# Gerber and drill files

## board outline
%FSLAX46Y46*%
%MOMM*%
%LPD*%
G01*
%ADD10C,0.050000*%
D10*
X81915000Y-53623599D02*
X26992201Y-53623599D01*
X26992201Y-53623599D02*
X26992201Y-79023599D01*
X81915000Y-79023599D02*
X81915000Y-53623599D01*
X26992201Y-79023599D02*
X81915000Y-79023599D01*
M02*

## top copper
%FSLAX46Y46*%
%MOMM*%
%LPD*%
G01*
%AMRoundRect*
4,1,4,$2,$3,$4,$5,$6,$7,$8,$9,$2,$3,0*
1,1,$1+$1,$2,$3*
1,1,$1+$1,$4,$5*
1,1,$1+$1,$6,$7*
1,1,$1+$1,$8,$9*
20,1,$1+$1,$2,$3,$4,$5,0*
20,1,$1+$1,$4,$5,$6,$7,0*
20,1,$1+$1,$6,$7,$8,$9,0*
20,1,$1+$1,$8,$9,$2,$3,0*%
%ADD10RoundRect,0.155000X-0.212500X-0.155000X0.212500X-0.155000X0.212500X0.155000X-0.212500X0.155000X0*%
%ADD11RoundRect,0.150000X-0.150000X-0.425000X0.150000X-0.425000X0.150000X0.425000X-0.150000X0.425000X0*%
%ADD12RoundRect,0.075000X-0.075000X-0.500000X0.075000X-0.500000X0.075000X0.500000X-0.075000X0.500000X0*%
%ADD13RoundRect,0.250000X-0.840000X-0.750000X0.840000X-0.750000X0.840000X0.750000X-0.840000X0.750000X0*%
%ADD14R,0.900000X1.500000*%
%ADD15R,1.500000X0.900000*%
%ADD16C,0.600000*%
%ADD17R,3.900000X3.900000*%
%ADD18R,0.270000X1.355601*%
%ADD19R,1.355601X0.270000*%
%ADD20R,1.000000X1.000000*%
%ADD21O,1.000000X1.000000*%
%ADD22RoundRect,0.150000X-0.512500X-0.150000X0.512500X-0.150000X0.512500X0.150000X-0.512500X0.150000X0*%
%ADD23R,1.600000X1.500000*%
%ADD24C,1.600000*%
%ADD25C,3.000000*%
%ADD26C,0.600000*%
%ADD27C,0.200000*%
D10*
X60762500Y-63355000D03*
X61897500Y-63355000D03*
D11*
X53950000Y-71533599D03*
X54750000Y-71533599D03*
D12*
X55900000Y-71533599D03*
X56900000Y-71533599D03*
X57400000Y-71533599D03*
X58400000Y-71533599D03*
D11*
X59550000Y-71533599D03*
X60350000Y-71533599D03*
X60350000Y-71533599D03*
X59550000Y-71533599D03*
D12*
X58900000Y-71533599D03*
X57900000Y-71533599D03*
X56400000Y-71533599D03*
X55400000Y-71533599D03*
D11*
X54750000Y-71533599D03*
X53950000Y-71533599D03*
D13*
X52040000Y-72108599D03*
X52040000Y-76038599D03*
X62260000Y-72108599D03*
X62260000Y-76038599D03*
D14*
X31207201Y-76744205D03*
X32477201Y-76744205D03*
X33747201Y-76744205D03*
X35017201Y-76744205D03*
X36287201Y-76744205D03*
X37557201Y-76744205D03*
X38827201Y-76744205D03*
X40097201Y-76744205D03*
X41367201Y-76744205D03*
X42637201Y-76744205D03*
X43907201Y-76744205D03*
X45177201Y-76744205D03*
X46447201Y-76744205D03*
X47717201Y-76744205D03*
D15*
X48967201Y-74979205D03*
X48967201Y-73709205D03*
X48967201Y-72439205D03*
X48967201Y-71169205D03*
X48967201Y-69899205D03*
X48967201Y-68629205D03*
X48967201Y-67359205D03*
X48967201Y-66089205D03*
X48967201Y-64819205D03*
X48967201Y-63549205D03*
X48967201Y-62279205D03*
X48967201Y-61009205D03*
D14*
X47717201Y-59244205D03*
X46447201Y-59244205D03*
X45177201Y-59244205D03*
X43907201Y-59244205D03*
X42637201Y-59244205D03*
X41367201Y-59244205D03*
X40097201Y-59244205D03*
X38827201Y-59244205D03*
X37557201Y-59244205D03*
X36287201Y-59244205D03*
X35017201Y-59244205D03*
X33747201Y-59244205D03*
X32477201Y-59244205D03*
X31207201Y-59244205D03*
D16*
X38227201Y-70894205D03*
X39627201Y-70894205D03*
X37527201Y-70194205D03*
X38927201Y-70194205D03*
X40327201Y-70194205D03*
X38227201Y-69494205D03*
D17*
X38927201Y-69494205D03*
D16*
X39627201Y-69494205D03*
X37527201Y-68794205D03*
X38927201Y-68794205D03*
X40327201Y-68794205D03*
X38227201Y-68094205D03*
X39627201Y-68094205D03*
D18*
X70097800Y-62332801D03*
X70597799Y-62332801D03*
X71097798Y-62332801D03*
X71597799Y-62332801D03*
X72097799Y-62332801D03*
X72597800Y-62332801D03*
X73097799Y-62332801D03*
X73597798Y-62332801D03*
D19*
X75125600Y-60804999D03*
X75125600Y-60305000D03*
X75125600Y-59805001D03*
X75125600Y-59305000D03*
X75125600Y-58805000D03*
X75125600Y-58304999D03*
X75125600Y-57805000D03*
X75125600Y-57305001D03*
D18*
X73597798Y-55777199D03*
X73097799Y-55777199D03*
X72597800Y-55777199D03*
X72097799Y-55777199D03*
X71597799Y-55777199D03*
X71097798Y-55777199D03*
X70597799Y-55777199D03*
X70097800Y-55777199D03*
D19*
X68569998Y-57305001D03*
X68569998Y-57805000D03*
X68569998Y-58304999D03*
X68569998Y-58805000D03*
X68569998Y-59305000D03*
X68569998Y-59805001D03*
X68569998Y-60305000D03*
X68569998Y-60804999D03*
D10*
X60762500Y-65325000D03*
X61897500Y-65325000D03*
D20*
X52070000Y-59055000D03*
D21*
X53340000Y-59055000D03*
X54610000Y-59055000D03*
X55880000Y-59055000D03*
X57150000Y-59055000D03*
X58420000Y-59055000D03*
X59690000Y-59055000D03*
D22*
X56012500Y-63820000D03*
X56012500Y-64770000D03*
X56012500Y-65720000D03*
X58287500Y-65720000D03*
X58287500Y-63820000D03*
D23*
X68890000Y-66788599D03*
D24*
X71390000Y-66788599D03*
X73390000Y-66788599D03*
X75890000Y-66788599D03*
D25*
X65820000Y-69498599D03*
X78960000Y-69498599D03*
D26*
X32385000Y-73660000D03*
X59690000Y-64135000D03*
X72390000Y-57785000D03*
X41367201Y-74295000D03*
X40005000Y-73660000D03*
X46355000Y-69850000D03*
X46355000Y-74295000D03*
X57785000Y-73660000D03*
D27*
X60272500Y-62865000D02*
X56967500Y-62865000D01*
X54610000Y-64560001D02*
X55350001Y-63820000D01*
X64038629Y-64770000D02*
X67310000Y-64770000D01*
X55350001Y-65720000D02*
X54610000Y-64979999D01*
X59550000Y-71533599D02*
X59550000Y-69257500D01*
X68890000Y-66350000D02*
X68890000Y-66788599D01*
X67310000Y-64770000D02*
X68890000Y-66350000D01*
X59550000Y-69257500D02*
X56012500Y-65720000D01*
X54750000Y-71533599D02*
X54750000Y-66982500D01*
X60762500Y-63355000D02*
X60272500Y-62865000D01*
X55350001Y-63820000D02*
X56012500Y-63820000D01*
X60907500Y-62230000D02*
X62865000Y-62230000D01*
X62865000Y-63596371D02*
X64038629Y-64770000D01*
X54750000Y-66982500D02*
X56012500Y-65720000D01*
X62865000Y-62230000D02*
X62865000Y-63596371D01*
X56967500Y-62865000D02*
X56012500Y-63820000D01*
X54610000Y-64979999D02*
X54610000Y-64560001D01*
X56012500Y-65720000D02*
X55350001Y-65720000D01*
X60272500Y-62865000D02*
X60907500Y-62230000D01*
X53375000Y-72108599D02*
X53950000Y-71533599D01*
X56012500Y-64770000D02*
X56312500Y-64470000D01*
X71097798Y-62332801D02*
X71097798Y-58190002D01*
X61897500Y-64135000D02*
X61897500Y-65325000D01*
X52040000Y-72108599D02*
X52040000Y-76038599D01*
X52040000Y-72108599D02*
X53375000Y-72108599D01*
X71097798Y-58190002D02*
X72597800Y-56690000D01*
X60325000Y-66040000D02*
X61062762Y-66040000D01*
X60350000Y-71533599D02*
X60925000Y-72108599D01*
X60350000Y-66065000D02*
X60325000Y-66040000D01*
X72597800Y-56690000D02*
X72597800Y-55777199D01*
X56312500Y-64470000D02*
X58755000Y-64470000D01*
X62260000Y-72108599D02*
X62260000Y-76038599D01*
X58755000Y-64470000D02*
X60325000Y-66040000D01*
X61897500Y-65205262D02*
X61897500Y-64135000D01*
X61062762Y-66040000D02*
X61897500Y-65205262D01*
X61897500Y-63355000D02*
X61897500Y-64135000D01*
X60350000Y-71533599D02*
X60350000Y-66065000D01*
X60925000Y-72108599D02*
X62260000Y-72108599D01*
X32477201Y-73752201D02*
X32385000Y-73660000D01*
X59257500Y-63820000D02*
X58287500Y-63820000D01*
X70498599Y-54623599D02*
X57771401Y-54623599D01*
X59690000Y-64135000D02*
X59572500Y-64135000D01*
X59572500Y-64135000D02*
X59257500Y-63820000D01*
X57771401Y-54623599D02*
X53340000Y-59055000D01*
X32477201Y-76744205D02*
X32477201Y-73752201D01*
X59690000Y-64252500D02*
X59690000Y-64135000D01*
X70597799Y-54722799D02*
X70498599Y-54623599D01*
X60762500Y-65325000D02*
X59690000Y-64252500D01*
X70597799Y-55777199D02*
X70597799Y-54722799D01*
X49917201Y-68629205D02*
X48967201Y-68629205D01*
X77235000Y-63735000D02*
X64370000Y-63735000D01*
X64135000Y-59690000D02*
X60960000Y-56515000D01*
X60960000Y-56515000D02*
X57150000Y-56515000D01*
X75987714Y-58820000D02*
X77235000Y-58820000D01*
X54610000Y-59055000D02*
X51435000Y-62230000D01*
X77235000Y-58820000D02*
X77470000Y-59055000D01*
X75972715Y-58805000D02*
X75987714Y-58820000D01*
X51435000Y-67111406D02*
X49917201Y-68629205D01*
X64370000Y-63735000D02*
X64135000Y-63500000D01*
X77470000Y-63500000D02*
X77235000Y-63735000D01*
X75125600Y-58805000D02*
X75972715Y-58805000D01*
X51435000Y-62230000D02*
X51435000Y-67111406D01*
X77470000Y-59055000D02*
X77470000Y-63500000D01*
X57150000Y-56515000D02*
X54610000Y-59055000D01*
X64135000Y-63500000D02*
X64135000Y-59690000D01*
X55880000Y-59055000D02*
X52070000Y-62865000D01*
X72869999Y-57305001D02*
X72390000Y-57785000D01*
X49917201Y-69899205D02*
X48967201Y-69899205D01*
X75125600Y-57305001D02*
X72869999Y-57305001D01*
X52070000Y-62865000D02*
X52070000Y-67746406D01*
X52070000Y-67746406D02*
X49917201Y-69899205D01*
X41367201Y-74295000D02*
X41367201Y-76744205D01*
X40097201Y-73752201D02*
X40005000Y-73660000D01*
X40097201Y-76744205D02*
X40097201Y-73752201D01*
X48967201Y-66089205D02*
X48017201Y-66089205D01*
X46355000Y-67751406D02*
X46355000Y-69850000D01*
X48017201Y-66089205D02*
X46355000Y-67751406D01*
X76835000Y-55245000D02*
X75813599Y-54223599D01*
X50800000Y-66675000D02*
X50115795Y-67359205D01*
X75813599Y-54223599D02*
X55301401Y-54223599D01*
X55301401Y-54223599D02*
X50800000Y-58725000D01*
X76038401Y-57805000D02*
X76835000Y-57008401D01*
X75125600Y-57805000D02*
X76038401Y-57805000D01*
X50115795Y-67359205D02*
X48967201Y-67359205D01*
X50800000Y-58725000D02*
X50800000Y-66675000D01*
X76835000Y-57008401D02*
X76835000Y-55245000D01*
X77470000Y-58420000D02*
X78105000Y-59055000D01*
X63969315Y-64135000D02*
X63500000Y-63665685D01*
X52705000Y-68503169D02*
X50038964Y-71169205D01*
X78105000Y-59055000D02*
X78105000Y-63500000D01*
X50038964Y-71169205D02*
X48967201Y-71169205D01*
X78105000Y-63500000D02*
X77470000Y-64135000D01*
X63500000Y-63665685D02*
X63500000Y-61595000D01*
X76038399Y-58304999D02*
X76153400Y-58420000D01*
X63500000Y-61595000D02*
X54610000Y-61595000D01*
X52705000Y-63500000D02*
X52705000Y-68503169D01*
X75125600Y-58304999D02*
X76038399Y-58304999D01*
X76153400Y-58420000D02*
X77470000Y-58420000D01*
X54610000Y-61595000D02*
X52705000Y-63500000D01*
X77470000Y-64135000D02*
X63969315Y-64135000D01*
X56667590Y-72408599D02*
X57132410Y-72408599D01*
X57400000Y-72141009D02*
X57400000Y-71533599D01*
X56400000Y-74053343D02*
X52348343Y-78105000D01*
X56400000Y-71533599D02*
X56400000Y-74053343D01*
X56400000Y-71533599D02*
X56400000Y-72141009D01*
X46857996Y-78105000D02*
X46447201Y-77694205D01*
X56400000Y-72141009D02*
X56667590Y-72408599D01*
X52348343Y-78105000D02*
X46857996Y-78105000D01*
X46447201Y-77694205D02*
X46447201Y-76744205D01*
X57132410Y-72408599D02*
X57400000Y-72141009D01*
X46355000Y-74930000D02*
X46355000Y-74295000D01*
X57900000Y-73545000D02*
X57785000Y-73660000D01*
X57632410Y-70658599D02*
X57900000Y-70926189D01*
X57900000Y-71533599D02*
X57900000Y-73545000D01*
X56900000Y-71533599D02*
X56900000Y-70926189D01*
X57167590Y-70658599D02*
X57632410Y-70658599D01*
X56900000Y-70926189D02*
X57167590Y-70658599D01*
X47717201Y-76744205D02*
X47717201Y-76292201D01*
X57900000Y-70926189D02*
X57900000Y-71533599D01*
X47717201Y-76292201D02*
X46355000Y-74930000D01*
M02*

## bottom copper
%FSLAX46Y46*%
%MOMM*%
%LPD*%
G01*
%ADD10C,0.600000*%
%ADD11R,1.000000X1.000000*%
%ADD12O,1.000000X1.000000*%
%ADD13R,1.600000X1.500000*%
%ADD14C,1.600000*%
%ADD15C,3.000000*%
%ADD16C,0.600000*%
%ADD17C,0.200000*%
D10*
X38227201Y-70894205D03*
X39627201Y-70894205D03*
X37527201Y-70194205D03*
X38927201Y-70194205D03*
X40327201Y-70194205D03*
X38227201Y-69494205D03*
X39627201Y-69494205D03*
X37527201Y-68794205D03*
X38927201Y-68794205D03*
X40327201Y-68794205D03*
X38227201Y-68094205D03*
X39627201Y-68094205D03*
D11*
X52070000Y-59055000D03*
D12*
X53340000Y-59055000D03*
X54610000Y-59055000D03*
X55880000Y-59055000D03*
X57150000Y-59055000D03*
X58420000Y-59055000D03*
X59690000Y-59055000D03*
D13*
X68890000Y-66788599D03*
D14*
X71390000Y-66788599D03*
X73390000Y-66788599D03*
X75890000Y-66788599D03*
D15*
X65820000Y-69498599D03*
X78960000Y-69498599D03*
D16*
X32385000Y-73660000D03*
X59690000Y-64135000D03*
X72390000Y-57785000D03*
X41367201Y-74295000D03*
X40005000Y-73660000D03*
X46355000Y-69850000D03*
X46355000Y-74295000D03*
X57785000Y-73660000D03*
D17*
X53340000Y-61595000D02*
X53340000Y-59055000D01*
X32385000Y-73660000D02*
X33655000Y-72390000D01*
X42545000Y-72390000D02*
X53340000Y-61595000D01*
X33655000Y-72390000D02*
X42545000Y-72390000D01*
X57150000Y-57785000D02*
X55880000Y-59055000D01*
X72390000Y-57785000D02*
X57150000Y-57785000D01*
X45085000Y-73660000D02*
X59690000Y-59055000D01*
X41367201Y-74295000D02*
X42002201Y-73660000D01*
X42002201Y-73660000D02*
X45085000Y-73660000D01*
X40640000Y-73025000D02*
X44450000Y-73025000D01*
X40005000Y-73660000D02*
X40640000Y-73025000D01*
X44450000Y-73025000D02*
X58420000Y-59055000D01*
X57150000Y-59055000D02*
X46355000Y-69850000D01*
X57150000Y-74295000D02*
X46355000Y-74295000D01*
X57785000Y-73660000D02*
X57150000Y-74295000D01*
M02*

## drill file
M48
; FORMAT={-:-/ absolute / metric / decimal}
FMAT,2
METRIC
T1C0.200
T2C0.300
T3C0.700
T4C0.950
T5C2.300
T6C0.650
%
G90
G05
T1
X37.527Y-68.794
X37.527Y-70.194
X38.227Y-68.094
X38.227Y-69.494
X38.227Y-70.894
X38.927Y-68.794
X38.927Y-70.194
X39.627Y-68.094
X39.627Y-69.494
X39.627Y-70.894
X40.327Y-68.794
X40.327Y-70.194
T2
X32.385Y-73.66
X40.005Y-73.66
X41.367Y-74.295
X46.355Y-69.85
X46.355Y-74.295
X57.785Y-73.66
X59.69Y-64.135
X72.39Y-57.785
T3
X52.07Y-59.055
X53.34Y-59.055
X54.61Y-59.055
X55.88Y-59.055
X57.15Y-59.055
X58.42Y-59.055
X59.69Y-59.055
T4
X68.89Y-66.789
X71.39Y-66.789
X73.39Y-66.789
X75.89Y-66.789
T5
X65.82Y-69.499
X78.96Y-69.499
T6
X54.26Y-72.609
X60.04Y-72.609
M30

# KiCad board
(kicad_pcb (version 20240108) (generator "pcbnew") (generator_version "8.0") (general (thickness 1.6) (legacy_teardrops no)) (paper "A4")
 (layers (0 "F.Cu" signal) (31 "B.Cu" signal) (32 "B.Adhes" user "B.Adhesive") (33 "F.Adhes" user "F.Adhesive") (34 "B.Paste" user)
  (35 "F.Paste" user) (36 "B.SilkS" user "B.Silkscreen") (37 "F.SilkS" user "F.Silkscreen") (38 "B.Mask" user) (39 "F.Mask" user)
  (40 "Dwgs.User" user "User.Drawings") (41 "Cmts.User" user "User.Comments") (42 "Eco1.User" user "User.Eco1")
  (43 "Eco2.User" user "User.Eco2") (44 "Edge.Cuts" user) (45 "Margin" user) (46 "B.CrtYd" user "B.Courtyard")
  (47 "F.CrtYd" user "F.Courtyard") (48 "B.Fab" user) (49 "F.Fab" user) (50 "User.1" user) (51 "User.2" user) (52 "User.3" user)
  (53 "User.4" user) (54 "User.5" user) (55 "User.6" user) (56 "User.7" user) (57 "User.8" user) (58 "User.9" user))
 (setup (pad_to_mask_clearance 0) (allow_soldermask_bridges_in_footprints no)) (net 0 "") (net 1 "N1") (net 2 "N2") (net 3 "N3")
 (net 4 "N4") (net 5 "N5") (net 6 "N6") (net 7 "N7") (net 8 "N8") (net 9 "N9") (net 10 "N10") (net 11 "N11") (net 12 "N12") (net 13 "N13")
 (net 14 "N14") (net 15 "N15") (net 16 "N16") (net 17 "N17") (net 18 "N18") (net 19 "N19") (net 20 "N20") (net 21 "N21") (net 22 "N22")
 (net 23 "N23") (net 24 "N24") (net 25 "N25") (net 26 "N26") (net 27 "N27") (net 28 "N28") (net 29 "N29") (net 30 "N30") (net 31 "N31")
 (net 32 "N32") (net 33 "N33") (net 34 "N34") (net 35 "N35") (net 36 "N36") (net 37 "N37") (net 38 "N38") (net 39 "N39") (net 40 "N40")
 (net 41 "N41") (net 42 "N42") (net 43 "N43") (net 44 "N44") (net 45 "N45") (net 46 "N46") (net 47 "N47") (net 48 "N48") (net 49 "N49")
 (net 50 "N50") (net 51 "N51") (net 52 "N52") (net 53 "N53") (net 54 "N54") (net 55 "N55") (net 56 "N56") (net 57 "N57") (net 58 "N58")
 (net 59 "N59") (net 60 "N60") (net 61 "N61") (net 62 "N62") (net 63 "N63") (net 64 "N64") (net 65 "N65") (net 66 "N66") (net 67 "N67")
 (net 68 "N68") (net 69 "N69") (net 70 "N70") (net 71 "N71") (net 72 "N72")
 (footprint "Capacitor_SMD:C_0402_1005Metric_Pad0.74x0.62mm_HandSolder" (layer "F.Cu") (at 61.33 63.355)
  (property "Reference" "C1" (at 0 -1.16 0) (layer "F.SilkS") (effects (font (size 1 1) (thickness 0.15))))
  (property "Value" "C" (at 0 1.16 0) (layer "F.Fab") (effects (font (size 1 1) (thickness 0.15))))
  (pad "1" smd roundrect (at -0.5675 0) (size 0.735 0.62) (layers "F.Cu" "F.Paste" "F.Mask") (roundrect_rratio 0.25) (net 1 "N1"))
  (pad "2" smd roundrect (at 0.5675 0) (size 0.735 0.62) (layers "F.Cu" "F.Paste" "F.Mask") (roundrect_rratio 0.25) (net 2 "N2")))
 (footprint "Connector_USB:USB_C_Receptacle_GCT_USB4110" (layer "F.Cu") (at 57.15 75.213599)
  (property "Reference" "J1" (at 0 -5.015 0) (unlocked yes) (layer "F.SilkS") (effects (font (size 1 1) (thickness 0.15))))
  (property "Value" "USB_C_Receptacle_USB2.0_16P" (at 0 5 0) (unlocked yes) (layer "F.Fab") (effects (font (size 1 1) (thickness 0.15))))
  (pad "" np_thru_hole circle (at -2.89 -2.605) (size 0.65 0.65) (drill 0.65) (layers "F&B.Cu" "*.Mask"))
  (pad "" np_thru_hole circle (at 2.89 -2.605) (size 0.65 0.65) (drill 0.65) (layers "F&B.Cu" "*.Mask"))
  (pad "A1" smd roundrect (at -3.2 -3.68) (size 0.6 1.15) (layers "F.Cu" "F.Paste" "F.Mask") (roundrect_rratio 0.25) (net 2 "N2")
   (thermal_bridge_angle 45))
  (pad "A4" smd roundrect (at -2.4 -3.68) (size 0.6 1.15) (layers "F.Cu" "F.Paste" "F.Mask") (roundrect_rratio 0.25) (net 1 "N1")
   (thermal_bridge_angle 45))
  (pad "A5" smd roundrect (at -1.25 -3.68) (size 0.3 1.15) (layers "F.Cu" "F.Paste" "F.Mask") (roundrect_rratio 0.25) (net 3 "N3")
   (thermal_bridge_angle 45))
  (pad "A6" smd roundrect (at -0.25 -3.68) (size 0.3 1.15) (layers "F.Cu" "F.Paste" "F.Mask") (roundrect_rratio 0.25) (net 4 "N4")
   (thermal_bridge_angle 45))
  (pad "A7" smd roundrect (at 0.25 -3.68) (size 0.3 1.15) (layers "F.Cu" "F.Paste" "F.Mask") (roundrect_rratio 0.25) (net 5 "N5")
   (thermal_bridge_angle 45))
  (pad "A8" smd roundrect (at 1.25 -3.68) (size 0.3 1.15) (layers "F.Cu" "F.Paste" "F.Mask") (roundrect_rratio 0.25) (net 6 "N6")
   (thermal_bridge_angle 45))
  (pad "A9" smd roundrect (at 2.4 -3.68) (size 0.6 1.15) (layers "F.Cu" "F.Paste" "F.Mask") (roundrect_rratio 0.25) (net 1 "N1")
   (thermal_bridge_angle 45))
  (pad "A12" smd roundrect (at 3.2 -3.68) (size 0.6 1.15) (layers "F.Cu" "F.Paste" "F.Mask") (roundrect_rratio 0.25) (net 2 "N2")
   (thermal_bridge_angle 45))
  (pad "B1" smd roundrect (at 3.2 -3.68) (size 0.6 1.15) (layers "F.Cu" "F.Paste" "F.Mask") (roundrect_rratio 0.25) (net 2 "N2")
   (thermal_bridge_angle 45))
  (pad "B4" smd roundrect (at 2.4 -3.68) (size 0.6 1.15) (layers "F.Cu" "F.Paste" "F.Mask") (roundrect_rratio 0.25) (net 1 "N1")
   (thermal_bridge_angle 45))
  (pad "B5" smd roundrect (at 1.75 -3.68) (size 0.3 1.15) (layers "F.Cu" "F.Paste" "F.Mask") (roundrect_rratio 0.25) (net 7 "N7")
   (thermal_bridge_angle 45))
  (pad "B6" smd roundrect (at 0.75 -3.68) (size 0.3 1.15) (layers "F.Cu" "F.Paste" "F.Mask") (roundrect_rratio 0.25) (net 4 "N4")
   (thermal_bridge_angle 45))
  (pad "B7" smd roundrect (at -0.75 -3.68) (size 0.3 1.15) (layers "F.Cu" "F.Paste" "F.Mask") (roundrect_rratio 0.25) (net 5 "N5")
   (thermal_bridge_angle 45))
  (pad "B8" smd roundrect (at -1.75 -3.68) (size 0.3 1.15) (layers "F.Cu" "F.Paste" "F.Mask") (roundrect_rratio 0.25) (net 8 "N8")
   (thermal_bridge_angle 45))
  (pad "B9" smd roundrect (at -2.4 -3.68) (size 0.6 1.15) (layers "F.Cu" "F.Paste" "F.Mask") (roundrect_rratio 0.25) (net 1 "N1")
   (thermal_bridge_angle 45))
  (pad "B12" smd roundrect (at -3.2 -3.68) (size 0.6 1.15) (layers "F.Cu" "F.Paste" "F.Mask") (roundrect_rratio 0.25) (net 2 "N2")
   (thermal_bridge_angle 45))
  (pad "S1" smd roundrect (at -5.11 -3.105) (size 2.18 2) (layers "F.Cu" "F.Paste" "F.Mask") (roundrect_rratio 0.125) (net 2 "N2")
   (thermal_bridge_angle 45))
  (pad "S1" smd roundrect (at -5.11 0.825) (size 2.18 2) (layers "F.Cu" "F.Paste" "F.Mask") (roundrect_rratio 0.125) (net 2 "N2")
   (thermal_bridge_angle 45))
  (pad "S1" smd roundrect (at 5.11 -3.105) (size 2.18 2) (layers "F.Cu" "F.Paste" "F.Mask") (roundrect_rratio 0.125) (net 2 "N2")
   (thermal_bridge_angle 45))
  (pad "S1" smd roundrect (at 5.11 0.825) (size 2.18 2) (layers "F.Cu" "F.Paste" "F.Mask") (roundrect_rratio 0.125) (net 2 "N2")
   (thermal_bridge_angle 45)))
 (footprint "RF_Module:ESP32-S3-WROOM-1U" (layer "F.Cu") (at 39.617201 67.994205 90)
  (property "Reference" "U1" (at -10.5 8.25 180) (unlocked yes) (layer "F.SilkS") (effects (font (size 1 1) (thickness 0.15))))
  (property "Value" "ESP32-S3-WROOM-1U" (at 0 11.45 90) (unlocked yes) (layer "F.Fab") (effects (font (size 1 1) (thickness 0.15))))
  (pad "" smd rect (at -2.904394 0.71 90) (size 0.9 0.9) (layers "F.Paste"))
  (pad "" smd rect (at -2.9 -2.09 90) (size 0.9 0.9) (layers "F.Paste"))
  (pad "" smd rect (at -2.9 -0.69 90) (size 0.9 0.9) (layers "F.Paste"))
  (pad "" smd rect (at -1.504394 0.71 90) (size 0.9 0.9) (layers "F.Paste"))
  (pad "" smd rect (at -1.5 -2.09 90) (size 0.9 0.9) (layers "F.Paste"))
  (pad "" smd rect (at -1.5 -0.69 90) (size 0.9 0.9) (layers "F.Paste"))
  (pad "" smd rect (at -0.104394 0.71 90) (size 0.9 0.9) (layers "F.Paste"))
  (pad "" smd rect (at -0.1 -2.09 90) (size 0.9 0.9) (layers "F.Paste"))
  (pad "" smd rect (at -0.1 -0.69 90) (size 0.9 0.9) (layers "F.Paste"))
  (pad "1" smd rect (at -8.75 -8.41 90) (size 1.5 0.9) (layers "F.Cu" "F.Paste" "F.Mask") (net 2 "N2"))
  (pad "2" smd rect (at -8.75 -7.14 90) (size 1.5 0.9) (layers "F.Cu" "F.Paste" "F.Mask") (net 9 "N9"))
  (pad "3" smd rect (at -8.75 -5.87 90) (size 1.5 0.9) (layers "F.Cu" "F.Paste" "F.Mask") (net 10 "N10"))
  (pad "4" smd rect (at -8.75 -4.6 90) (size 1.5 0.9) (layers "F.Cu" "F.Paste" "F.Mask") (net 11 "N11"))
  (pad "5" smd rect (at -8.75 -3.33 90) (size 1.5 0.9) (layers "F.Cu" "F.Paste" "F.Mask") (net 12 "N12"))
  (pad "6" smd rect (at -8.75 -2.06 90) (size 1.5 0.9) (layers "F.Cu" "F.Paste" "F.Mask") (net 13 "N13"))
  (pad "7" smd rect (at -8.75 -0.79 90) (size 1.5 0.9) (layers "F.Cu" "F.Paste" "F.Mask") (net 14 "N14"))
  (pad "8" smd rect (at -8.75 0.48 90) (size 1.5 0.9) (layers "F.Cu" "F.Paste" "F.Mask") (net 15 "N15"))
  (pad "9" smd rect (at -8.75 1.75 90) (size 1.5 0.9) (layers "F.Cu" "F.Paste" "F.Mask") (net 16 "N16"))
  (pad "10" smd rect (at -8.75 3.02 90) (size 1.5 0.9) (layers "F.Cu" "F.Paste" "F.Mask") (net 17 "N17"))
  (pad "11" smd rect (at -8.75 4.29 90) (size 1.5 0.9) (layers "F.Cu" "F.Paste" "F.Mask") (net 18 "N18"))
  (pad "12" smd rect (at -8.75 5.56 90) (size 1.5 0.9) (layers "F.Cu" "F.Paste" "F.Mask") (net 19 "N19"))
  (pad "13" smd rect (at -8.75 6.83 90) (size 1.5 0.9) (layers "F.Cu" "F.Paste" "F.Mask") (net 5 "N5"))
  (pad "14" smd rect (at -8.75 8.1 270) (size 1.5 0.9) (layers "F.Cu" "F.Paste" "F.Mask") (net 4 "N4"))
  (pad "15" smd rect (at -6.985 9.35) (size 1.5 0.9) (layers "F.Cu" "F.Paste" "F.Mask") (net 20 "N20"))
  (pad "16" smd rect (at -5.715 9.35) (size 1.5 0.9) (layers "F.Cu" "F.Paste" "F.Mask") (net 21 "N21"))
  (pad "17" smd rect (at -4.445 9.35) (size 1.5 0.9) (layers "F.Cu" "F.Paste" "F.Mask") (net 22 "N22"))
  (pad "18" smd rect (at -3.175 9.35) (size 1.5 0.9) (layers "F.Cu" "F.Paste" "F.Mask") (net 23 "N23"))
  (pad "19" smd rect (at -1.905 9.35) (size 1.5 0.9) (layers "F.Cu" "F.Paste" "F.Mask") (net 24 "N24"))
  (pad "20" smd rect (at -0.635 9.35) (size 1.5 0.9) (layers "F.Cu" "F.Paste" "F.Mask") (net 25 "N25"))
  (pad "21" smd rect (at 0.635 9.35) (size 1.5 0.9) (layers "F.Cu" "F.Paste" "F.Mask") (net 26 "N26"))
  (pad "22" smd rect (at 1.905 9.35) (size 1.5 0.9) (layers "F.Cu" "F.Paste" "F.Mask") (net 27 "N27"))
  (pad "23" smd rect (at 3.175 9.35) (size 1.5 0.9) (layers "F.Cu" "F.Paste" "F.Mask") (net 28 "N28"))
  (pad "24" smd rect (at 4.445 9.35) (size 1.5 0.9) (layers "F.Cu" "F.Paste" "F.Mask") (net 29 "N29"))
  (pad "25" smd rect (at 5.715 9.35) (size 1.5 0.9) (layers "F.Cu" "F.Paste" "F.Mask") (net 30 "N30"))
  (pad "26" smd rect (at 6.985 9.35) (size 1.5 0.9) (layers "F.Cu" "F.Paste" "F.Mask") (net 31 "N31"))
  (pad "27" smd rect (at 8.75 8.1 90) (size 1.5 0.9) (layers "F.Cu" "F.Paste" "F.Mask") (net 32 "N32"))
  (pad "28" smd rect (at 8.75 6.83 90) (size 1.5 0.9) (layers "F.Cu" "F.Paste" "F.Mask") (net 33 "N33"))
  (pad "29" smd rect (at 8.75 5.56 90) (size 1.5 0.9) (layers "F.Cu" "F.Paste" "F.Mask") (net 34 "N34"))
  (pad "30" smd rect (at 8.75 4.29 90) (size 1.5 0.9) (layers "F.Cu" "F.Paste" "F.Mask") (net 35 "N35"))
  (pad "31" smd rect (at 8.75 3.02 90) (size 1.5 0.9) (layers "F.Cu" "F.Paste" "F.Mask") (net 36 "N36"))
  (pad "32" smd rect (at 8.75 1.75 90) (size 1.5 0.9) (layers "F.Cu" "F.Paste" "F.Mask") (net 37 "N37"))
  (pad "33" smd rect (at 8.75 0.48 90) (size 1.5 0.9) (layers "F.Cu" "F.Paste" "F.Mask") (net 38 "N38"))
  (pad "34" smd rect (at 8.75 -0.79 90) (size 1.5 0.9) (layers "F.Cu" "F.Paste" "F.Mask") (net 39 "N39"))
  (pad "35" smd rect (at 8.75 -2.06 90) (size 1.5 0.9) (layers "F.Cu" "F.Paste" "F.Mask") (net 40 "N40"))
  (pad "36" smd rect (at 8.75 -3.33 90) (size 1.5 0.9) (layers "F.Cu" "F.Paste" "F.Mask") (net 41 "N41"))
  (pad "37" smd rect (at 8.75 -4.6 90) (size 1.5 0.9) (layers "F.Cu" "F.Paste" "F.Mask") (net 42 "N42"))
  (pad "38" smd rect (at 8.75 -5.87 90) (size 1.5 0.9) (layers "F.Cu" "F.Paste" "F.Mask") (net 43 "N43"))
  (pad "39" smd rect (at 8.75 -7.14 90) (size 1.5 0.9) (layers "F.Cu" "F.Paste" "F.Mask") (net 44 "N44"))
  (pad "40" smd rect (at 8.75 -8.41 90) (size 1.5 0.9) (layers "F.Cu" "F.Paste" "F.Mask") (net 2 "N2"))
  (pad "41" thru_hole circle (at -2.9 -1.39 90) (size 0.6 0.6) (drill 0.2) (layers "*.Cu" "F.Mask") (remove_unused_layers no) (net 2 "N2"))
  (pad "41" thru_hole circle (at -2.9 0.01 90) (size 0.6 0.6) (drill 0.2) (layers "*.Cu" "F.Mask") (remove_unused_layers no) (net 2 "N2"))
  (pad "41" thru_hole circle (at -2.2 -2.09 90) (size 0.6 0.6) (drill 0.2) (layers "*.Cu" "F.Mask") (remove_unused_layers no) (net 2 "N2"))
  (pad "41" thru_hole circle (at -2.2 -0.69 90) (size 0.6 0.6) (drill 0.2) (layers "*.Cu" "F.Mask") (remove_unused_layers no) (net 2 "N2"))
  (pad "41" thru_hole circle (at -2.2 0.71 90) (size 0.6 0.6) (drill 0.2) (layers "*.Cu" "F.Mask") (remove_unused_layers no) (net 2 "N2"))
  (pad "41" thru_hole circle (at -1.5 -1.39 90) (size 0.6 0.6) (drill 0.2) (layers "*.Cu" "F.Mask") (remove_unused_layers no) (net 2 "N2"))
  (pad "41" smd rect (at -1.5 -0.69 90) (size 3.9 3.9) (layers "F.Cu" "F.Mask") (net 2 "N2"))
  (pad "41" thru_hole circle (at -1.5 0.01 90) (size 0.6 0.6) (drill 0.2) (layers "*.Cu" "F.Mask") (remove_unused_layers no) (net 2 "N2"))
  (pad "41" thru_hole circle (at -0.8 -2.09 90) (size 0.6 0.6) (drill 0.2) (layers "*.Cu" "F.Mask") (remove_unused_layers no) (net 2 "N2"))
  (pad "41" thru_hole circle (at -0.8 -0.69 180) (size 0.6 0.6) (drill 0.2) (layers "*.Cu" "F.Mask") (remove_unused_layers no) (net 2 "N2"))
  (pad "41" thru_hole circle (at -0.8 0.71 90) (size 0.6 0.6) (drill 0.2) (layers "*.Cu" "F.Mask") (remove_unused_layers no) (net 2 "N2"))
  (pad "41" thru_hole circle (at -0.1 -1.39 90) (size 0.6 0.6) (drill 0.2) (layers "*.Cu" "F.Mask") (remove_unused_layers no) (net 2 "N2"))
  (pad "41" thru_hole circle (at -0.1 0.01 90) (size 0.6 0.6) (drill 0.2) (layers "*.Cu" "F.Mask") (remove_unused_layers no) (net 2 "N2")))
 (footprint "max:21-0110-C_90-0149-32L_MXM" (layer "F.Cu") (at 71.847799 59.055 90)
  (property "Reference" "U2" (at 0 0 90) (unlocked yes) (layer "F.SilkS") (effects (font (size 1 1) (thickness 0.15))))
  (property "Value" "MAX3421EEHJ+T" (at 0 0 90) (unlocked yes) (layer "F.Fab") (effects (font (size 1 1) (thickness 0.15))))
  (pad "1" smd rect (at -3.277801 -1.749999 180) (size 0.27 1.355601) (layers "F.Cu" "F.Paste" "F.Mask") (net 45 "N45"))
  (pad "2" smd rect (at -3.277801 -1.25 180) (size 0.27 1.355601) (layers "F.Cu" "F.Paste" "F.Mask") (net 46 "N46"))
  (pad "3" smd rect (at -3.277801 -0.750001 180) (size 0.27 1.355601) (layers "F.Cu" "F.Paste" "F.Mask") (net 2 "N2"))
  (pad "4" smd rect (at -3.277801 -0.25 180) (size 0.27 1.355601) (layers "F.Cu" "F.Paste" "F.Mask") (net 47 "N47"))
  (pad "5" smd rect (at -3.277801 0.25 180) (size 0.27 1.355601) (layers "F.Cu" "F.Paste" "F.Mask") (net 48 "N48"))
  (pad "6" smd rect (at -3.277801 0.750001 180) (size 0.27 1.355601) (layers "F.Cu" "F.Paste" "F.Mask") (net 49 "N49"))
  (pad "7" smd rect (at -3.277801 1.25 180) (size 0.27 1.355601) (layers "F.Cu" "F.Paste" "F.Mask") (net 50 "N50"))
  (pad "8" smd rect (at -3.277801 1.749999 180) (size 0.27 1.355601) (layers "F.Cu" "F.Paste" "F.Mask") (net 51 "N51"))
  (pad "9" smd rect (at -1.749999 3.277801 90) (size 0.27 1.355601) (layers "F.Cu" "F.Paste" "F.Mask") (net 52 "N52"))
  (pad "10" smd rect (at -1.25 3.277801 90) (size 0.27 1.355601) (layers "F.Cu" "F.Paste" "F.Mask") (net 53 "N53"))
  (pad "11" smd rect (at -0.750001 3.277801 90) (size 0.27 1.355601) (layers "F.Cu" "F.Paste" "F.Mask") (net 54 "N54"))
  (pad "12" smd rect (at -0.25 3.277801 90) (size 0.27 1.355601) (layers "F.Cu" "F.Paste" "F.Mask") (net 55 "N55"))
  (pad "13" smd rect (at 0.25 3.277801 90) (size 0.27 1.355601) (layers "F.Cu" "F.Paste" "F.Mask") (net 25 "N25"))
  (pad "14" smd rect (at 0.750001 3.277801 90) (size 0.27 1.355601) (layers "F.Cu" "F.Paste" "F.Mask") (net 23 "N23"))
  (pad "15" smd rect (at 1.25 3.277801 90) (size 0.27 1.355601) (layers "F.Cu" "F.Paste" "F.Mask") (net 26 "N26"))
  (pad "16" smd rect (at 1.749999 3.277801 90) (size 0.27 1.355601) (layers "F.Cu" "F.Paste" "F.Mask") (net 24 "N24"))
  (pad "17" smd rect (at 3.277801 1.749999 180) (size 0.27 1.355601) (layers "F.Cu" "F.Paste" "F.Mask") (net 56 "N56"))
  (pad "18" smd rect (at 3.277801 1.25 180) (size 0.27 1.355601) (layers "F.Cu" "F.Paste" "F.Mask") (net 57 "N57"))
  (pad "19" smd rect (at 3.277801 0.750001 180) (size 0.27 1.355601) (layers "F.Cu" "F.Paste" "F.Mask") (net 2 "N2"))
  (pad "20" smd rect (at 3.277801 0.25 180) (size 0.27 1.355601) (layers "F.Cu" "F.Paste" "F.Mask") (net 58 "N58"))
  (pad "21" smd rect (at 3.277801 -0.25 180) (size 0.27 1.355601) (layers "F.Cu" "F.Paste" "F.Mask") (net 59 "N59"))
  (pad "22" smd rect (at 3.277801 -0.750001 180) (size 0.27 1.355601) (layers "F.Cu" "F.Paste" "F.Mask") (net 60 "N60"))
  (pad "23" smd rect (at 3.277801 -1.25 180) (size 0.27 1.355601) (layers "F.Cu" "F.Paste" "F.Mask") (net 9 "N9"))
  (pad "24" smd rect (at 3.277801 -1.749999 180) (size 0.27 1.355601) (layers "F.Cu" "F.Paste" "F.Mask") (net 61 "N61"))
  (pad "25" smd rect (at 1.749999 -3.277801 90) (size 0.27 1.355601) (layers "F.Cu" "F.Paste" "F.Mask") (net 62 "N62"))
  (pad "26" smd rect (at 1.25 -3.277801 90) (size 0.27 1.355601) (layers "F.Cu" "F.Paste" "F.Mask") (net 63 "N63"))
  (pad "27" smd rect (at 0.750001 -3.277801 90) (size 0.27 1.355601) (layers "F.Cu" "F.Paste" "F.Mask") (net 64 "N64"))
  (pad "28" smd rect (at 0.25 -3.277801 90) (size 0.27 1.355601) (layers "F.Cu" "F.Paste" "F.Mask") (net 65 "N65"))
  (pad "29" smd rect (at -0.25 -3.277801 90) (size 0.27 1.355601) (layers "F.Cu" "F.Paste" "F.Mask") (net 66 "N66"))
  (pad "30" smd rect (at -0.750001 -3.277801 90) (size 0.27 1.355601) (layers "F.Cu" "F.Paste" "F.Mask") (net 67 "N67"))
  (pad "31" smd rect (at -1.25 -3.277801 90) (size 0.27 1.355601) (layers "F.Cu" "F.Paste" "F.Mask") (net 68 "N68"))
  (pad "32" smd rect (at -1.749999 -3.277801 90) (size 0.27 1.355601) (layers "F.Cu" "F.Paste" "F.Mask") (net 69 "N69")))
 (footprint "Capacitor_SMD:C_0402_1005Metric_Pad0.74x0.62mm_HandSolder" (layer "F.Cu") (at 61.33 65.325)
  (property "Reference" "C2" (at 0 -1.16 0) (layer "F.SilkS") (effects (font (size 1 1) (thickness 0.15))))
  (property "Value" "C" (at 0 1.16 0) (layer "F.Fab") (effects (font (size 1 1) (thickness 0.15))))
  (pad "1" smd roundrect (at -0.5675 0) (size 0.735 0.62) (layers "F.Cu" "F.Paste" "F.Mask") (roundrect_rratio 0.25) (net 9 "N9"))
  (pad "2" smd roundrect (at 0.5675 0) (size 0.735 0.62) (layers "F.Cu" "F.Paste" "F.Mask") (roundrect_rratio 0.25) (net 2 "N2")))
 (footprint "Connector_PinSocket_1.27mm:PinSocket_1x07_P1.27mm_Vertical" (layer "F.Cu") (at 55.895 55.28)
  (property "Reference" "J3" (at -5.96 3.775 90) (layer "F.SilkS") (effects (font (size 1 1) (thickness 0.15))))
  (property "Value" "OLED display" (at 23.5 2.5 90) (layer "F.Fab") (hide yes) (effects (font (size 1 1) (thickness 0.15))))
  (pad "1" thru_hole rect (at -3.825 3.775 90) (size 1 1) (drill 0.7) (layers "*.Cu" "*.Mask") (remove_unused_layers no) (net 2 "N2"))
  (pad "2" thru_hole oval (at -2.555 3.775 90) (size 1 1) (drill 0.7) (layers "*.Cu" "*.Mask") (remove_unused_layers no) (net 9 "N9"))
  (pad "3" thru_hole oval (at -1.285 3.775 90) (size 1 1) (drill 0.7) (layers "*.Cu" "*.Mask") (remove_unused_layers no) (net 25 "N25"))
  (pad "4" thru_hole oval (at -0.015 3.775 90) (size 1 1) (drill 0.7) (layers "*.Cu" "*.Mask") (remove_unused_layers no) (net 24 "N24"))
  (pad "5" thru_hole oval (at 1.255 3.775 90) (size 1 1) (drill 0.7) (layers "*.Cu" "*.Mask") (remove_unused_layers no) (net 27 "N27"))
  (pad "6" thru_hole oval (at 2.525 3.775 90) (size 1 1) (drill 0.7) (layers "*.Cu" "*.Mask") (remove_unused_layers no) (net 15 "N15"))
  (pad "7" thru_hole oval (at 3.795 3.775 90) (size 1 1) (drill 0.7) (layers "*.Cu" "*.Mask") (remove_unused_layers no) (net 16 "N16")))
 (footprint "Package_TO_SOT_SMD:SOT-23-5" (layer "F.Cu") (at 57.15 64.77)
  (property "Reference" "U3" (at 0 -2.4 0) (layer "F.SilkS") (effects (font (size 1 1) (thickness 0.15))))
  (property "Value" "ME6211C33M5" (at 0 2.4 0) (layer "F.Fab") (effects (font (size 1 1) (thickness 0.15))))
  (pad "1" smd roundrect (at -1.1375 -0.95) (size 1.325 0.6) (layers "F.Cu" "F.Paste" "F.Mask") (roundrect_rratio 0.25) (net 1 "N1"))
  (pad "2" smd roundrect (at -1.1375 0) (size 1.325 0.6) (layers "F.Cu" "F.Paste" "F.Mask") (roundrect_rratio 0.25) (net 2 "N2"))
  (pad "3" smd roundrect (at -1.1375 0.95) (size 1.325 0.6) (layers "F.Cu" "F.Paste" "F.Mask") (roundrect_rratio 0.25) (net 1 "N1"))
  (pad "4" smd roundrect (at 1.1375 0.95) (size 1.325 0.6) (layers "F.Cu" "F.Paste" "F.Mask") (roundrect_rratio 0.25) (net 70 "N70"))
  (pad "5" smd roundrect (at 1.1375 -0.95) (size 1.325 0.6) (layers "F.Cu" "F.Paste" "F.Mask") (roundrect_rratio 0.25) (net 9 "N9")))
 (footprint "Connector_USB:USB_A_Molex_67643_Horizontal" (layer "F.Cu") (at 68.89 66.788599)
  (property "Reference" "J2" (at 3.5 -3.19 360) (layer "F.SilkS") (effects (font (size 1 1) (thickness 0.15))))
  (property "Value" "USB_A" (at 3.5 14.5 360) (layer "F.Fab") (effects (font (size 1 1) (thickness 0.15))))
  (pad "1" thru_hole rect (at 0 0) (size 1.6 1.5) (drill 0.95) (layers "*.Cu" "*.Mask") (remove_unused_layers no) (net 1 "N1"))
  (pad "2" thru_hole circle (at 2.5 0) (size 1.6 1.6) (drill 0.95) (layers "*.Cu" "*.Mask") (remove_unused_layers no) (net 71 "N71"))
  (pad "3" thru_hole circle (at 4.5 0) (size 1.6 1.6) (drill 0.95) (layers "*.Cu" "*.Mask") (remove_unused_layers no) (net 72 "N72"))
  (pad "4" thru_hole circle (at 7 0) (size 1.6 1.6) (drill 0.95) (layers "*.Cu" "*.Mask") (remove_unused_layers no) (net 2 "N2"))
  (pad "5" thru_hole circle (at -3.07 2.71) (size 3 3) (drill 2.3) (layers "*.Cu" "*.Mask") (remove_unused_layers no) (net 2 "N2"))
  (pad "5" thru_hole circle (at 10.07 2.71) (size 3 3) (drill 2.3) (layers "*.Cu" "*.Mask") (remove_unused_layers no) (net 2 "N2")))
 (gr_line (start 81.915 53.623599) (end 26.992201 53.623599) (stroke (width 0.05) (type default)) (layer "Edge.Cuts"))
 (gr_line (start 26.992201 53.623599) (end 26.992201 79.023599) (stroke (width 0.05) (type default)) (layer "Edge.Cuts"))
 (gr_line (start 81.915 79.023599) (end 81.915 53.623599) (stroke (width 0.05) (type default)) (layer "Edge.Cuts"))
 (gr_line (start 26.992201 79.023599) (end 81.915 79.023599) (stroke (width 0.05) (type default)) (layer "Edge.Cuts"))
 (segment (start 60.2725 62.865) (end 56.9675 62.865) (width 0.2) (layer "F.Cu") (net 1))
 (segment (start 54.61 64.560001) (end 55.350001 63.82) (width 0.2) (layer "F.Cu") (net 1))
 (segment (start 64.038629 64.77) (end 67.31 64.77) (width 0.2) (layer "F.Cu") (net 1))
 (segment (start 55.350001 65.72) (end 54.61 64.979999) (width 0.2) (layer "F.Cu") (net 1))
 (segment (start 59.55 71.533599) (end 59.55 69.2575) (width 0.2) (layer "F.Cu") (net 1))
 (segment (start 68.89 66.35) (end 68.89 66.788599) (width 0.2) (layer "F.Cu") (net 1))
 (segment (start 67.31 64.77) (end 68.89 66.35) (width 0.2) (layer "F.Cu") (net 1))
 (segment (start 59.55 69.2575) (end 56.0125 65.72) (width 0.2) (layer "F.Cu") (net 1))
 (segment (start 54.75 71.533599) (end 54.75 66.9825) (width 0.2) (layer "F.Cu") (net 1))
 (segment (start 60.7625 63.355) (end 60.2725 62.865) (width 0.2) (layer "F.Cu") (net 1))
 (segment (start 55.350001 63.82) (end 56.0125 63.82) (width 0.2) (layer "F.Cu") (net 1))
 (segment (start 60.9075 62.23) (end 62.865 62.23) (width 0.2) (layer "F.Cu") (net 1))
 (segment (start 62.865 63.596371) (end 64.038629 64.77) (width 0.2) (layer "F.Cu") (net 1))
 (segment (start 54.75 66.9825) (end 56.0125 65.72) (width 0.2) (layer "F.Cu") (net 1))
 (segment (start 62.865 62.23) (end 62.865 63.596371) (width 0.2) (layer "F.Cu") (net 1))
 (segment (start 56.9675 62.865) (end 56.0125 63.82) (width 0.2) (layer "F.Cu") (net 1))
 (segment (start 54.61 64.979999) (end 54.61 64.560001) (width 0.2) (layer "F.Cu") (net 1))
 (segment (start 56.0125 65.72) (end 55.350001 65.72) (width 0.2) (layer "F.Cu") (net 1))
 (segment (start 60.2725 62.865) (end 60.9075 62.23) (width 0.2) (layer "F.Cu") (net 1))
 (segment (start 53.375 72.108599) (end 53.95 71.533599) (width 0.2) (layer "F.Cu") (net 2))
 (segment (start 56.0125 64.77) (end 56.3125 64.47) (width 0.2) (layer "F.Cu") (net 2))
 (segment (start 71.097798 62.332801) (end 71.097798 58.190002) (width 0.2) (layer "F.Cu") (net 2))
 (segment (start 61.8975 64.135) (end 61.8975 65.325) (width 0.2) (layer "F.Cu") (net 2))
 (segment (start 52.04 72.108599) (end 52.04 76.038599) (width 0.2) (layer "F.Cu") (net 2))
 (segment (start 52.04 72.108599) (end 53.375 72.108599) (width 0.2) (layer "F.Cu") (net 2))
 (segment (start 71.097798 58.190002) (end 72.5978 56.69) (width 0.2) (layer "F.Cu") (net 2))
 (segment (start 60.325 66.04) (end 61.062762 66.04) (width 0.2) (layer "F.Cu") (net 2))
 (segment (start 60.35 71.533599) (end 60.925 72.108599) (width 0.2) (layer "F.Cu") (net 2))
 (segment (start 60.35 66.065) (end 60.325 66.04) (width 0.2) (layer "F.Cu") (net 2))
 (segment (start 72.5978 56.69) (end 72.5978 55.777199) (width 0.2) (layer "F.Cu") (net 2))
 (segment (start 56.3125 64.47) (end 58.755 64.47) (width 0.2) (layer "F.Cu") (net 2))
 (segment (start 62.26 72.108599) (end 62.26 76.038599) (width 0.2) (layer "F.Cu") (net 2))
 (segment (start 58.755 64.47) (end 60.325 66.04) (width 0.2) (layer "F.Cu") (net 2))
 (segment (start 61.8975 65.205262) (end 61.8975 64.135) (width 0.2) (layer "F.Cu") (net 2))
 (segment (start 61.062762 66.04) (end 61.8975 65.205262) (width 0.2) (layer "F.Cu") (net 2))
 (segment (start 61.8975 63.355) (end 61.8975 64.135) (width 0.2) (layer "F.Cu") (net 2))
 (segment (start 60.35 71.533599) (end 60.35 66.065) (width 0.2) (layer "F.Cu") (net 2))
 (segment (start 60.925 72.108599) (end 62.26 72.108599) (width 0.2) (layer "F.Cu") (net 2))
 (segment (start 32.477201 73.752201) (end 32.385 73.66) (width 0.2) (layer "F.Cu") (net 9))
 (segment (start 59.2575 63.82) (end 58.2875 63.82) (width 0.2) (layer "F.Cu") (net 9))
 (segment (start 70.498599 54.623599) (end 57.771401 54.623599) (width 0.2) (layer "F.Cu") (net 9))
 (segment (start 59.69 64.135) (end 59.5725 64.135) (width 0.2) (layer "F.Cu") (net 9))
 (segment (start 59.5725 64.135) (end 59.2575 63.82) (width 0.2) (layer "F.Cu") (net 9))
 (segment (start 57.771401 54.623599) (end 53.34 59.055) (width 0.2) (layer "F.Cu") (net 9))
 (segment (start 32.477201 76.744205) (end 32.477201 73.752201) (width 0.2) (layer "F.Cu") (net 9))
 (segment (start 59.69 64.2525) (end 59.69 64.135) (width 0.2) (layer "F.Cu") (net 9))
 (segment (start 70.597799 54.722799) (end 70.498599 54.623599) (width 0.2) (layer "F.Cu") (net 9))
 (segment (start 60.7625 65.325) (end 59.69 64.2525) (width 0.2) (layer "F.Cu") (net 9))
 (segment (start 70.597799 55.777199) (end 70.597799 54.722799) (width 0.2) (layer "F.Cu") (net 9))
 (via (at 32.385 73.66) (size 0.6) (drill 0.3) (layers "F.Cu" "B.Cu") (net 9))
 (via (at 59.69 64.135) (size 0.6) (drill 0.3) (layers "F.Cu" "B.Cu") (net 9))
 (segment (start 53.34 61.595) (end 53.34 59.055) (width 0.2) (layer "B.Cu") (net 9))
 (segment (start 32.385 73.66) (end 33.655 72.39) (width 0.2) (layer "B.Cu") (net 9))
 (segment (start 42.545 72.39) (end 53.34 61.595) (width 0.2) (layer "B.Cu") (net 9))
 (segment (start 33.655 72.39) (end 42.545 72.39) (width 0.2) (layer "B.Cu") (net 9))
 (segment (start 49.917201 68.629205) (end 48.967201 68.629205) (width 0.2) (layer "F.Cu") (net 25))
 (segment (start 77.235 63.735) (end 64.37 63.735) (width 0.2) (layer "F.Cu") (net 25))
 (segment (start 64.135 59.69) (end 60.96 56.515) (width 0.2) (layer "F.Cu") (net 25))
 (segment (start 60.96 56.515) (end 57.15 56.515) (width 0.2) (layer "F.Cu") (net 25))
 (segment (start 75.987714 58.82) (end 77.235 58.82) (width 0.2) (layer "F.Cu") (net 25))
 (segment (start 54.61 59.055) (end 51.435 62.23) (width 0.2) (layer "F.Cu") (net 25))
 (segment (start 77.235 58.82) (end 77.47 59.055) (width 0.2) (layer "F.Cu") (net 25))
 (segment (start 75.972715 58.805) (end 75.987714 58.82) (width 0.2) (layer "F.Cu") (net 25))
 (segment (start 51.435 67.111406) (end 49.917201 68.629205) (width 0.2) (layer "F.Cu") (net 25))
 (segment (start 64.37 63.735) (end 64.135 63.5) (width 0.2) (layer "F.Cu") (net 25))
 (segment (start 77.47 63.5) (end 77.235 63.735) (width 0.2) (layer "F.Cu") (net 25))
 (segment (start 75.1256 58.805) (end 75.972715 58.805) (width 0.2) (layer "F.Cu") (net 25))
 (segment (start 51.435 62.23) (end 51.435 67.111406) (width 0.2) (layer "F.Cu") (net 25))
 (segment (start 77.47 59.055) (end 77.47 63.5) (width 0.2) (layer "F.Cu") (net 25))
 (segment (start 57.15 56.515) (end 54.61 59.055) (width 0.2) (layer "F.Cu") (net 25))
 (segment (start 64.135 63.5) (end 64.135 59.69) (width 0.2) (layer "F.Cu") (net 25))
 (segment (start 55.88 59.055) (end 52.07 62.865) (width 0.2) (layer "F.Cu") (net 24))
 (segment (start 72.869999 57.305001) (end 72.39 57.785) (width 0.2) (layer "F.Cu") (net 24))
 (segment (start 49.917201 69.899205) (end 48.967201 69.899205) (width 0.2) (layer "F.Cu") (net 24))
 (segment (start 75.1256 57.305001) (end 72.869999 57.305001) (width 0.2) (layer "F.Cu") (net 24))
 (segment (start 52.07 62.865) (end 52.07 67.746406) (width 0.2) (layer "F.Cu") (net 24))
 (segment (start 52.07 67.746406) (end 49.917201 69.899205) (width 0.2) (layer "F.Cu") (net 24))
 (via (at 72.39 57.785) (size 0.6) (drill 0.3) (layers "F.Cu" "B.Cu") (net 24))
 (segment (start 57.15 57.785) (end 55.88 59.055) (width 0.2) (layer "B.Cu") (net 24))
 (segment (start 72.39 57.785) (end 57.15 57.785) (width 0.2) (layer "B.Cu") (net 24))
 (segment (start 41.367201 74.295) (end 41.367201 76.744205) (width 0.2) (layer "F.Cu") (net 16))
 (via (at 41.367201 74.295) (size 0.6) (drill 0.3) (layers "F.Cu" "B.Cu") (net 16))
 (segment (start 45.085 73.66) (end 59.69 59.055) (width 0.2) (layer "B.Cu") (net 16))
 (segment (start 41.367201 74.295) (end 42.002201 73.66) (width 0.2) (layer "B.Cu") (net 16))
 (segment (start 42.002201 73.66) (end 45.085 73.66) (width 0.2) (layer "B.Cu") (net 16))
 (segment (start 40.097201 73.752201) (end 40.005 73.66) (width 0.2) (layer "F.Cu") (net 15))
 (segment (start 40.097201 76.744205) (end 40.097201 73.752201) (width 0.2) (layer "F.Cu") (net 15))
 (via (at 40.005 73.66) (size 0.6) (drill 0.3) (layers "F.Cu" "B.Cu") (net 15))
 (segment (start 40.64 73.025) (end 44.45 73.025) (width 0.2) (layer "B.Cu") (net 15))
 (segment (start 40.005 73.66) (end 40.64 73.025) (width 0.2) (layer "B.Cu") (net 15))
 (segment (start 44.45 73.025) (end 58.42 59.055) (width 0.2) (layer "B.Cu") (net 15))
 (segment (start 48.967201 66.089205) (end 48.017201 66.089205) (width 0.2) (layer "F.Cu") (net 27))
 (segment (start 46.355 67.751406) (end 46.355 69.85) (width 0.2) (layer "F.Cu") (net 27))
 (segment (start 48.017201 66.089205) (end 46.355 67.751406) (width 0.2) (layer "F.Cu") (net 27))
 (via (at 46.355 69.85) (size 0.6) (drill 0.3) (layers "F.Cu" "B.Cu") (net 27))
 (segment (start 57.15 59.055) (end 46.355 69.85) (width 0.2) (layer "B.Cu") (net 27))
 (segment (start 76.835 55.245) (end 75.813599 54.223599) (width 0.2) (layer "F.Cu") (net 26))
 (segment (start 50.8 66.675) (end 50.115795 67.359205) (width 0.2) (layer "F.Cu") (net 26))
 (segment (start 75.813599 54.223599) (end 55.301401 54.223599) (width 0.2) (layer "F.Cu") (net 26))
 (segment (start 55.301401 54.223599) (end 50.8 58.725) (width 0.2) (layer "F.Cu") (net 26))
 (segment (start 76.038401 57.805) (end 76.835 57.008401) (width 0.2) (layer "F.Cu") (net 26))
 (segment (start 75.1256 57.805) (end 76.038401 57.805) (width 0.2) (layer "F.Cu") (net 26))
 (segment (start 50.115795 67.359205) (end 48.967201 67.359205) (width 0.2) (layer "F.Cu") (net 26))
 (segment (start 50.8 58.725) (end 50.8 66.675) (width 0.2) (layer "F.Cu") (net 26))
 (segment (start 76.835 57.008401) (end 76.835 55.245) (width 0.2) (layer "F.Cu") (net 26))
 (segment (start 77.47 58.42) (end 78.105 59.055) (width 0.2) (layer "F.Cu") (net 23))
 (segment (start 63.969315 64.135) (end 63.5 63.665685) (width 0.2) (layer "F.Cu") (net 23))
 (segment (start 52.705 68.503169) (end 50.038964 71.169205) (width 0.2) (layer "F.Cu") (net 23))
 (segment (start 78.105 59.055) (end 78.105 63.5) (width 0.2) (layer "F.Cu") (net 23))
 (segment (start 50.038964 71.169205) (end 48.967201 71.169205) (width 0.2) (layer "F.Cu") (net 23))
 (segment (start 78.105 63.5) (end 77.47 64.135) (width 0.2) (layer "F.Cu") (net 23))
 (segment (start 63.5 63.665685) (end 63.5 61.595) (width 0.2) (layer "F.Cu") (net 23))
 (segment (start 76.038399 58.304999) (end 76.1534 58.42) (width 0.2) (layer "F.Cu") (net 23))
 (segment (start 63.5 61.595) (end 54.61 61.595) (width 0.2) (layer "F.Cu") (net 23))
 (segment (start 52.705 63.5) (end 52.705 68.503169) (width 0.2) (layer "F.Cu") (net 23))
 (segment (start 75.1256 58.304999) (end 76.038399 58.304999) (width 0.2) (layer "F.Cu") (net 23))
 (segment (start 76.1534 58.42) (end 77.47 58.42) (width 0.2) (layer "F.Cu") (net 23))
 (segment (start 54.61 61.595) (end 52.705 63.5) (width 0.2) (layer "F.Cu") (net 23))
 (segment (start 77.47 64.135) (end 63.969315 64.135) (width 0.2) (layer "F.Cu") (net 23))
 (segment (start 56.66759 72.408599) (end 57.13241 72.408599) (width 0.2) (layer "F.Cu") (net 5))
 (segment (start 57.4 72.141009) (end 57.4 71.533599) (width 0.2) (layer "F.Cu") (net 5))
 (segment (start 56.4 74.053343) (end 52.348343 78.105) (width 0.2) (layer "F.Cu") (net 5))
 (segment (start 56.4 71.533599) (end 56.4 74.053343) (width 0.2) (layer "F.Cu") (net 5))
 (segment (start 56.4 71.533599) (end 56.4 72.141009) (width 0.2) (layer "F.Cu") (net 5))
 (segment (start 46.857996 78.105) (end 46.447201 77.694205) (width 0.2) (layer "F.Cu") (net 5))
 (segment (start 56.4 72.141009) (end 56.66759 72.408599) (width 0.2) (layer "F.Cu") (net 5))
 (segment (start 52.348343 78.105) (end 46.857996 78.105) (width 0.2) (layer "F.Cu") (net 5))
 (segment (start 46.447201 77.694205) (end 46.447201 76.744205) (width 0.2) (layer "F.Cu") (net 5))
 (segment (start 57.13241 72.408599) (end 57.4 72.141009) (width 0.2) (layer "F.Cu") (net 5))
 (segment (start 46.355 74.93) (end 46.355 74.295) (width 0.2) (layer "F.Cu") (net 4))
 (segment (start 57.9 73.545) (end 57.785 73.66) (width 0.2) (layer "F.Cu") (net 4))
 (segment (start 57.63241 70.658599) (end 57.9 70.926189) (width 0.2) (layer "F.Cu") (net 4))
 (segment (start 57.9 71.533599) (end 57.9 73.545) (width 0.2) (layer "F.Cu") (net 4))
 (segment (start 56.9 71.533599) (end 56.9 70.926189) (width 0.2) (layer "F.Cu") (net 4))
 (segment (start 57.16759 70.658599) (end 57.63241 70.658599) (width 0.2) (layer "F.Cu") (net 4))
 (segment (start 56.9 70.926189) (end 57.16759 70.658599) (width 0.2) (layer "F.Cu") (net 4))
 (segment (start 47.717201 76.744205) (end 47.717201 76.292201) (width 0.2) (layer "F.Cu") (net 4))
 (segment (start 57.9 70.926189) (end 57.9 71.533599) (width 0.2) (layer "F.Cu") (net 4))
 (segment (start 47.717201 76.292201) (end 46.355 74.93) (width 0.2) (layer "F.Cu") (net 4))
 (via (at 46.355 74.295) (size 0.6) (drill 0.3) (layers "F.Cu" "B.Cu") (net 4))
 (via (at 57.785 73.66) (size 0.6) (drill 0.3) (layers "F.Cu" "B.Cu") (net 4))
 (segment (start 57.15 74.295) (end 46.355 74.295) (width 0.2) (layer "B.Cu") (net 4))
 (segment (start 57.785 73.66) (end 57.15 74.295) (width 0.2) (layer "B.Cu") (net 4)))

